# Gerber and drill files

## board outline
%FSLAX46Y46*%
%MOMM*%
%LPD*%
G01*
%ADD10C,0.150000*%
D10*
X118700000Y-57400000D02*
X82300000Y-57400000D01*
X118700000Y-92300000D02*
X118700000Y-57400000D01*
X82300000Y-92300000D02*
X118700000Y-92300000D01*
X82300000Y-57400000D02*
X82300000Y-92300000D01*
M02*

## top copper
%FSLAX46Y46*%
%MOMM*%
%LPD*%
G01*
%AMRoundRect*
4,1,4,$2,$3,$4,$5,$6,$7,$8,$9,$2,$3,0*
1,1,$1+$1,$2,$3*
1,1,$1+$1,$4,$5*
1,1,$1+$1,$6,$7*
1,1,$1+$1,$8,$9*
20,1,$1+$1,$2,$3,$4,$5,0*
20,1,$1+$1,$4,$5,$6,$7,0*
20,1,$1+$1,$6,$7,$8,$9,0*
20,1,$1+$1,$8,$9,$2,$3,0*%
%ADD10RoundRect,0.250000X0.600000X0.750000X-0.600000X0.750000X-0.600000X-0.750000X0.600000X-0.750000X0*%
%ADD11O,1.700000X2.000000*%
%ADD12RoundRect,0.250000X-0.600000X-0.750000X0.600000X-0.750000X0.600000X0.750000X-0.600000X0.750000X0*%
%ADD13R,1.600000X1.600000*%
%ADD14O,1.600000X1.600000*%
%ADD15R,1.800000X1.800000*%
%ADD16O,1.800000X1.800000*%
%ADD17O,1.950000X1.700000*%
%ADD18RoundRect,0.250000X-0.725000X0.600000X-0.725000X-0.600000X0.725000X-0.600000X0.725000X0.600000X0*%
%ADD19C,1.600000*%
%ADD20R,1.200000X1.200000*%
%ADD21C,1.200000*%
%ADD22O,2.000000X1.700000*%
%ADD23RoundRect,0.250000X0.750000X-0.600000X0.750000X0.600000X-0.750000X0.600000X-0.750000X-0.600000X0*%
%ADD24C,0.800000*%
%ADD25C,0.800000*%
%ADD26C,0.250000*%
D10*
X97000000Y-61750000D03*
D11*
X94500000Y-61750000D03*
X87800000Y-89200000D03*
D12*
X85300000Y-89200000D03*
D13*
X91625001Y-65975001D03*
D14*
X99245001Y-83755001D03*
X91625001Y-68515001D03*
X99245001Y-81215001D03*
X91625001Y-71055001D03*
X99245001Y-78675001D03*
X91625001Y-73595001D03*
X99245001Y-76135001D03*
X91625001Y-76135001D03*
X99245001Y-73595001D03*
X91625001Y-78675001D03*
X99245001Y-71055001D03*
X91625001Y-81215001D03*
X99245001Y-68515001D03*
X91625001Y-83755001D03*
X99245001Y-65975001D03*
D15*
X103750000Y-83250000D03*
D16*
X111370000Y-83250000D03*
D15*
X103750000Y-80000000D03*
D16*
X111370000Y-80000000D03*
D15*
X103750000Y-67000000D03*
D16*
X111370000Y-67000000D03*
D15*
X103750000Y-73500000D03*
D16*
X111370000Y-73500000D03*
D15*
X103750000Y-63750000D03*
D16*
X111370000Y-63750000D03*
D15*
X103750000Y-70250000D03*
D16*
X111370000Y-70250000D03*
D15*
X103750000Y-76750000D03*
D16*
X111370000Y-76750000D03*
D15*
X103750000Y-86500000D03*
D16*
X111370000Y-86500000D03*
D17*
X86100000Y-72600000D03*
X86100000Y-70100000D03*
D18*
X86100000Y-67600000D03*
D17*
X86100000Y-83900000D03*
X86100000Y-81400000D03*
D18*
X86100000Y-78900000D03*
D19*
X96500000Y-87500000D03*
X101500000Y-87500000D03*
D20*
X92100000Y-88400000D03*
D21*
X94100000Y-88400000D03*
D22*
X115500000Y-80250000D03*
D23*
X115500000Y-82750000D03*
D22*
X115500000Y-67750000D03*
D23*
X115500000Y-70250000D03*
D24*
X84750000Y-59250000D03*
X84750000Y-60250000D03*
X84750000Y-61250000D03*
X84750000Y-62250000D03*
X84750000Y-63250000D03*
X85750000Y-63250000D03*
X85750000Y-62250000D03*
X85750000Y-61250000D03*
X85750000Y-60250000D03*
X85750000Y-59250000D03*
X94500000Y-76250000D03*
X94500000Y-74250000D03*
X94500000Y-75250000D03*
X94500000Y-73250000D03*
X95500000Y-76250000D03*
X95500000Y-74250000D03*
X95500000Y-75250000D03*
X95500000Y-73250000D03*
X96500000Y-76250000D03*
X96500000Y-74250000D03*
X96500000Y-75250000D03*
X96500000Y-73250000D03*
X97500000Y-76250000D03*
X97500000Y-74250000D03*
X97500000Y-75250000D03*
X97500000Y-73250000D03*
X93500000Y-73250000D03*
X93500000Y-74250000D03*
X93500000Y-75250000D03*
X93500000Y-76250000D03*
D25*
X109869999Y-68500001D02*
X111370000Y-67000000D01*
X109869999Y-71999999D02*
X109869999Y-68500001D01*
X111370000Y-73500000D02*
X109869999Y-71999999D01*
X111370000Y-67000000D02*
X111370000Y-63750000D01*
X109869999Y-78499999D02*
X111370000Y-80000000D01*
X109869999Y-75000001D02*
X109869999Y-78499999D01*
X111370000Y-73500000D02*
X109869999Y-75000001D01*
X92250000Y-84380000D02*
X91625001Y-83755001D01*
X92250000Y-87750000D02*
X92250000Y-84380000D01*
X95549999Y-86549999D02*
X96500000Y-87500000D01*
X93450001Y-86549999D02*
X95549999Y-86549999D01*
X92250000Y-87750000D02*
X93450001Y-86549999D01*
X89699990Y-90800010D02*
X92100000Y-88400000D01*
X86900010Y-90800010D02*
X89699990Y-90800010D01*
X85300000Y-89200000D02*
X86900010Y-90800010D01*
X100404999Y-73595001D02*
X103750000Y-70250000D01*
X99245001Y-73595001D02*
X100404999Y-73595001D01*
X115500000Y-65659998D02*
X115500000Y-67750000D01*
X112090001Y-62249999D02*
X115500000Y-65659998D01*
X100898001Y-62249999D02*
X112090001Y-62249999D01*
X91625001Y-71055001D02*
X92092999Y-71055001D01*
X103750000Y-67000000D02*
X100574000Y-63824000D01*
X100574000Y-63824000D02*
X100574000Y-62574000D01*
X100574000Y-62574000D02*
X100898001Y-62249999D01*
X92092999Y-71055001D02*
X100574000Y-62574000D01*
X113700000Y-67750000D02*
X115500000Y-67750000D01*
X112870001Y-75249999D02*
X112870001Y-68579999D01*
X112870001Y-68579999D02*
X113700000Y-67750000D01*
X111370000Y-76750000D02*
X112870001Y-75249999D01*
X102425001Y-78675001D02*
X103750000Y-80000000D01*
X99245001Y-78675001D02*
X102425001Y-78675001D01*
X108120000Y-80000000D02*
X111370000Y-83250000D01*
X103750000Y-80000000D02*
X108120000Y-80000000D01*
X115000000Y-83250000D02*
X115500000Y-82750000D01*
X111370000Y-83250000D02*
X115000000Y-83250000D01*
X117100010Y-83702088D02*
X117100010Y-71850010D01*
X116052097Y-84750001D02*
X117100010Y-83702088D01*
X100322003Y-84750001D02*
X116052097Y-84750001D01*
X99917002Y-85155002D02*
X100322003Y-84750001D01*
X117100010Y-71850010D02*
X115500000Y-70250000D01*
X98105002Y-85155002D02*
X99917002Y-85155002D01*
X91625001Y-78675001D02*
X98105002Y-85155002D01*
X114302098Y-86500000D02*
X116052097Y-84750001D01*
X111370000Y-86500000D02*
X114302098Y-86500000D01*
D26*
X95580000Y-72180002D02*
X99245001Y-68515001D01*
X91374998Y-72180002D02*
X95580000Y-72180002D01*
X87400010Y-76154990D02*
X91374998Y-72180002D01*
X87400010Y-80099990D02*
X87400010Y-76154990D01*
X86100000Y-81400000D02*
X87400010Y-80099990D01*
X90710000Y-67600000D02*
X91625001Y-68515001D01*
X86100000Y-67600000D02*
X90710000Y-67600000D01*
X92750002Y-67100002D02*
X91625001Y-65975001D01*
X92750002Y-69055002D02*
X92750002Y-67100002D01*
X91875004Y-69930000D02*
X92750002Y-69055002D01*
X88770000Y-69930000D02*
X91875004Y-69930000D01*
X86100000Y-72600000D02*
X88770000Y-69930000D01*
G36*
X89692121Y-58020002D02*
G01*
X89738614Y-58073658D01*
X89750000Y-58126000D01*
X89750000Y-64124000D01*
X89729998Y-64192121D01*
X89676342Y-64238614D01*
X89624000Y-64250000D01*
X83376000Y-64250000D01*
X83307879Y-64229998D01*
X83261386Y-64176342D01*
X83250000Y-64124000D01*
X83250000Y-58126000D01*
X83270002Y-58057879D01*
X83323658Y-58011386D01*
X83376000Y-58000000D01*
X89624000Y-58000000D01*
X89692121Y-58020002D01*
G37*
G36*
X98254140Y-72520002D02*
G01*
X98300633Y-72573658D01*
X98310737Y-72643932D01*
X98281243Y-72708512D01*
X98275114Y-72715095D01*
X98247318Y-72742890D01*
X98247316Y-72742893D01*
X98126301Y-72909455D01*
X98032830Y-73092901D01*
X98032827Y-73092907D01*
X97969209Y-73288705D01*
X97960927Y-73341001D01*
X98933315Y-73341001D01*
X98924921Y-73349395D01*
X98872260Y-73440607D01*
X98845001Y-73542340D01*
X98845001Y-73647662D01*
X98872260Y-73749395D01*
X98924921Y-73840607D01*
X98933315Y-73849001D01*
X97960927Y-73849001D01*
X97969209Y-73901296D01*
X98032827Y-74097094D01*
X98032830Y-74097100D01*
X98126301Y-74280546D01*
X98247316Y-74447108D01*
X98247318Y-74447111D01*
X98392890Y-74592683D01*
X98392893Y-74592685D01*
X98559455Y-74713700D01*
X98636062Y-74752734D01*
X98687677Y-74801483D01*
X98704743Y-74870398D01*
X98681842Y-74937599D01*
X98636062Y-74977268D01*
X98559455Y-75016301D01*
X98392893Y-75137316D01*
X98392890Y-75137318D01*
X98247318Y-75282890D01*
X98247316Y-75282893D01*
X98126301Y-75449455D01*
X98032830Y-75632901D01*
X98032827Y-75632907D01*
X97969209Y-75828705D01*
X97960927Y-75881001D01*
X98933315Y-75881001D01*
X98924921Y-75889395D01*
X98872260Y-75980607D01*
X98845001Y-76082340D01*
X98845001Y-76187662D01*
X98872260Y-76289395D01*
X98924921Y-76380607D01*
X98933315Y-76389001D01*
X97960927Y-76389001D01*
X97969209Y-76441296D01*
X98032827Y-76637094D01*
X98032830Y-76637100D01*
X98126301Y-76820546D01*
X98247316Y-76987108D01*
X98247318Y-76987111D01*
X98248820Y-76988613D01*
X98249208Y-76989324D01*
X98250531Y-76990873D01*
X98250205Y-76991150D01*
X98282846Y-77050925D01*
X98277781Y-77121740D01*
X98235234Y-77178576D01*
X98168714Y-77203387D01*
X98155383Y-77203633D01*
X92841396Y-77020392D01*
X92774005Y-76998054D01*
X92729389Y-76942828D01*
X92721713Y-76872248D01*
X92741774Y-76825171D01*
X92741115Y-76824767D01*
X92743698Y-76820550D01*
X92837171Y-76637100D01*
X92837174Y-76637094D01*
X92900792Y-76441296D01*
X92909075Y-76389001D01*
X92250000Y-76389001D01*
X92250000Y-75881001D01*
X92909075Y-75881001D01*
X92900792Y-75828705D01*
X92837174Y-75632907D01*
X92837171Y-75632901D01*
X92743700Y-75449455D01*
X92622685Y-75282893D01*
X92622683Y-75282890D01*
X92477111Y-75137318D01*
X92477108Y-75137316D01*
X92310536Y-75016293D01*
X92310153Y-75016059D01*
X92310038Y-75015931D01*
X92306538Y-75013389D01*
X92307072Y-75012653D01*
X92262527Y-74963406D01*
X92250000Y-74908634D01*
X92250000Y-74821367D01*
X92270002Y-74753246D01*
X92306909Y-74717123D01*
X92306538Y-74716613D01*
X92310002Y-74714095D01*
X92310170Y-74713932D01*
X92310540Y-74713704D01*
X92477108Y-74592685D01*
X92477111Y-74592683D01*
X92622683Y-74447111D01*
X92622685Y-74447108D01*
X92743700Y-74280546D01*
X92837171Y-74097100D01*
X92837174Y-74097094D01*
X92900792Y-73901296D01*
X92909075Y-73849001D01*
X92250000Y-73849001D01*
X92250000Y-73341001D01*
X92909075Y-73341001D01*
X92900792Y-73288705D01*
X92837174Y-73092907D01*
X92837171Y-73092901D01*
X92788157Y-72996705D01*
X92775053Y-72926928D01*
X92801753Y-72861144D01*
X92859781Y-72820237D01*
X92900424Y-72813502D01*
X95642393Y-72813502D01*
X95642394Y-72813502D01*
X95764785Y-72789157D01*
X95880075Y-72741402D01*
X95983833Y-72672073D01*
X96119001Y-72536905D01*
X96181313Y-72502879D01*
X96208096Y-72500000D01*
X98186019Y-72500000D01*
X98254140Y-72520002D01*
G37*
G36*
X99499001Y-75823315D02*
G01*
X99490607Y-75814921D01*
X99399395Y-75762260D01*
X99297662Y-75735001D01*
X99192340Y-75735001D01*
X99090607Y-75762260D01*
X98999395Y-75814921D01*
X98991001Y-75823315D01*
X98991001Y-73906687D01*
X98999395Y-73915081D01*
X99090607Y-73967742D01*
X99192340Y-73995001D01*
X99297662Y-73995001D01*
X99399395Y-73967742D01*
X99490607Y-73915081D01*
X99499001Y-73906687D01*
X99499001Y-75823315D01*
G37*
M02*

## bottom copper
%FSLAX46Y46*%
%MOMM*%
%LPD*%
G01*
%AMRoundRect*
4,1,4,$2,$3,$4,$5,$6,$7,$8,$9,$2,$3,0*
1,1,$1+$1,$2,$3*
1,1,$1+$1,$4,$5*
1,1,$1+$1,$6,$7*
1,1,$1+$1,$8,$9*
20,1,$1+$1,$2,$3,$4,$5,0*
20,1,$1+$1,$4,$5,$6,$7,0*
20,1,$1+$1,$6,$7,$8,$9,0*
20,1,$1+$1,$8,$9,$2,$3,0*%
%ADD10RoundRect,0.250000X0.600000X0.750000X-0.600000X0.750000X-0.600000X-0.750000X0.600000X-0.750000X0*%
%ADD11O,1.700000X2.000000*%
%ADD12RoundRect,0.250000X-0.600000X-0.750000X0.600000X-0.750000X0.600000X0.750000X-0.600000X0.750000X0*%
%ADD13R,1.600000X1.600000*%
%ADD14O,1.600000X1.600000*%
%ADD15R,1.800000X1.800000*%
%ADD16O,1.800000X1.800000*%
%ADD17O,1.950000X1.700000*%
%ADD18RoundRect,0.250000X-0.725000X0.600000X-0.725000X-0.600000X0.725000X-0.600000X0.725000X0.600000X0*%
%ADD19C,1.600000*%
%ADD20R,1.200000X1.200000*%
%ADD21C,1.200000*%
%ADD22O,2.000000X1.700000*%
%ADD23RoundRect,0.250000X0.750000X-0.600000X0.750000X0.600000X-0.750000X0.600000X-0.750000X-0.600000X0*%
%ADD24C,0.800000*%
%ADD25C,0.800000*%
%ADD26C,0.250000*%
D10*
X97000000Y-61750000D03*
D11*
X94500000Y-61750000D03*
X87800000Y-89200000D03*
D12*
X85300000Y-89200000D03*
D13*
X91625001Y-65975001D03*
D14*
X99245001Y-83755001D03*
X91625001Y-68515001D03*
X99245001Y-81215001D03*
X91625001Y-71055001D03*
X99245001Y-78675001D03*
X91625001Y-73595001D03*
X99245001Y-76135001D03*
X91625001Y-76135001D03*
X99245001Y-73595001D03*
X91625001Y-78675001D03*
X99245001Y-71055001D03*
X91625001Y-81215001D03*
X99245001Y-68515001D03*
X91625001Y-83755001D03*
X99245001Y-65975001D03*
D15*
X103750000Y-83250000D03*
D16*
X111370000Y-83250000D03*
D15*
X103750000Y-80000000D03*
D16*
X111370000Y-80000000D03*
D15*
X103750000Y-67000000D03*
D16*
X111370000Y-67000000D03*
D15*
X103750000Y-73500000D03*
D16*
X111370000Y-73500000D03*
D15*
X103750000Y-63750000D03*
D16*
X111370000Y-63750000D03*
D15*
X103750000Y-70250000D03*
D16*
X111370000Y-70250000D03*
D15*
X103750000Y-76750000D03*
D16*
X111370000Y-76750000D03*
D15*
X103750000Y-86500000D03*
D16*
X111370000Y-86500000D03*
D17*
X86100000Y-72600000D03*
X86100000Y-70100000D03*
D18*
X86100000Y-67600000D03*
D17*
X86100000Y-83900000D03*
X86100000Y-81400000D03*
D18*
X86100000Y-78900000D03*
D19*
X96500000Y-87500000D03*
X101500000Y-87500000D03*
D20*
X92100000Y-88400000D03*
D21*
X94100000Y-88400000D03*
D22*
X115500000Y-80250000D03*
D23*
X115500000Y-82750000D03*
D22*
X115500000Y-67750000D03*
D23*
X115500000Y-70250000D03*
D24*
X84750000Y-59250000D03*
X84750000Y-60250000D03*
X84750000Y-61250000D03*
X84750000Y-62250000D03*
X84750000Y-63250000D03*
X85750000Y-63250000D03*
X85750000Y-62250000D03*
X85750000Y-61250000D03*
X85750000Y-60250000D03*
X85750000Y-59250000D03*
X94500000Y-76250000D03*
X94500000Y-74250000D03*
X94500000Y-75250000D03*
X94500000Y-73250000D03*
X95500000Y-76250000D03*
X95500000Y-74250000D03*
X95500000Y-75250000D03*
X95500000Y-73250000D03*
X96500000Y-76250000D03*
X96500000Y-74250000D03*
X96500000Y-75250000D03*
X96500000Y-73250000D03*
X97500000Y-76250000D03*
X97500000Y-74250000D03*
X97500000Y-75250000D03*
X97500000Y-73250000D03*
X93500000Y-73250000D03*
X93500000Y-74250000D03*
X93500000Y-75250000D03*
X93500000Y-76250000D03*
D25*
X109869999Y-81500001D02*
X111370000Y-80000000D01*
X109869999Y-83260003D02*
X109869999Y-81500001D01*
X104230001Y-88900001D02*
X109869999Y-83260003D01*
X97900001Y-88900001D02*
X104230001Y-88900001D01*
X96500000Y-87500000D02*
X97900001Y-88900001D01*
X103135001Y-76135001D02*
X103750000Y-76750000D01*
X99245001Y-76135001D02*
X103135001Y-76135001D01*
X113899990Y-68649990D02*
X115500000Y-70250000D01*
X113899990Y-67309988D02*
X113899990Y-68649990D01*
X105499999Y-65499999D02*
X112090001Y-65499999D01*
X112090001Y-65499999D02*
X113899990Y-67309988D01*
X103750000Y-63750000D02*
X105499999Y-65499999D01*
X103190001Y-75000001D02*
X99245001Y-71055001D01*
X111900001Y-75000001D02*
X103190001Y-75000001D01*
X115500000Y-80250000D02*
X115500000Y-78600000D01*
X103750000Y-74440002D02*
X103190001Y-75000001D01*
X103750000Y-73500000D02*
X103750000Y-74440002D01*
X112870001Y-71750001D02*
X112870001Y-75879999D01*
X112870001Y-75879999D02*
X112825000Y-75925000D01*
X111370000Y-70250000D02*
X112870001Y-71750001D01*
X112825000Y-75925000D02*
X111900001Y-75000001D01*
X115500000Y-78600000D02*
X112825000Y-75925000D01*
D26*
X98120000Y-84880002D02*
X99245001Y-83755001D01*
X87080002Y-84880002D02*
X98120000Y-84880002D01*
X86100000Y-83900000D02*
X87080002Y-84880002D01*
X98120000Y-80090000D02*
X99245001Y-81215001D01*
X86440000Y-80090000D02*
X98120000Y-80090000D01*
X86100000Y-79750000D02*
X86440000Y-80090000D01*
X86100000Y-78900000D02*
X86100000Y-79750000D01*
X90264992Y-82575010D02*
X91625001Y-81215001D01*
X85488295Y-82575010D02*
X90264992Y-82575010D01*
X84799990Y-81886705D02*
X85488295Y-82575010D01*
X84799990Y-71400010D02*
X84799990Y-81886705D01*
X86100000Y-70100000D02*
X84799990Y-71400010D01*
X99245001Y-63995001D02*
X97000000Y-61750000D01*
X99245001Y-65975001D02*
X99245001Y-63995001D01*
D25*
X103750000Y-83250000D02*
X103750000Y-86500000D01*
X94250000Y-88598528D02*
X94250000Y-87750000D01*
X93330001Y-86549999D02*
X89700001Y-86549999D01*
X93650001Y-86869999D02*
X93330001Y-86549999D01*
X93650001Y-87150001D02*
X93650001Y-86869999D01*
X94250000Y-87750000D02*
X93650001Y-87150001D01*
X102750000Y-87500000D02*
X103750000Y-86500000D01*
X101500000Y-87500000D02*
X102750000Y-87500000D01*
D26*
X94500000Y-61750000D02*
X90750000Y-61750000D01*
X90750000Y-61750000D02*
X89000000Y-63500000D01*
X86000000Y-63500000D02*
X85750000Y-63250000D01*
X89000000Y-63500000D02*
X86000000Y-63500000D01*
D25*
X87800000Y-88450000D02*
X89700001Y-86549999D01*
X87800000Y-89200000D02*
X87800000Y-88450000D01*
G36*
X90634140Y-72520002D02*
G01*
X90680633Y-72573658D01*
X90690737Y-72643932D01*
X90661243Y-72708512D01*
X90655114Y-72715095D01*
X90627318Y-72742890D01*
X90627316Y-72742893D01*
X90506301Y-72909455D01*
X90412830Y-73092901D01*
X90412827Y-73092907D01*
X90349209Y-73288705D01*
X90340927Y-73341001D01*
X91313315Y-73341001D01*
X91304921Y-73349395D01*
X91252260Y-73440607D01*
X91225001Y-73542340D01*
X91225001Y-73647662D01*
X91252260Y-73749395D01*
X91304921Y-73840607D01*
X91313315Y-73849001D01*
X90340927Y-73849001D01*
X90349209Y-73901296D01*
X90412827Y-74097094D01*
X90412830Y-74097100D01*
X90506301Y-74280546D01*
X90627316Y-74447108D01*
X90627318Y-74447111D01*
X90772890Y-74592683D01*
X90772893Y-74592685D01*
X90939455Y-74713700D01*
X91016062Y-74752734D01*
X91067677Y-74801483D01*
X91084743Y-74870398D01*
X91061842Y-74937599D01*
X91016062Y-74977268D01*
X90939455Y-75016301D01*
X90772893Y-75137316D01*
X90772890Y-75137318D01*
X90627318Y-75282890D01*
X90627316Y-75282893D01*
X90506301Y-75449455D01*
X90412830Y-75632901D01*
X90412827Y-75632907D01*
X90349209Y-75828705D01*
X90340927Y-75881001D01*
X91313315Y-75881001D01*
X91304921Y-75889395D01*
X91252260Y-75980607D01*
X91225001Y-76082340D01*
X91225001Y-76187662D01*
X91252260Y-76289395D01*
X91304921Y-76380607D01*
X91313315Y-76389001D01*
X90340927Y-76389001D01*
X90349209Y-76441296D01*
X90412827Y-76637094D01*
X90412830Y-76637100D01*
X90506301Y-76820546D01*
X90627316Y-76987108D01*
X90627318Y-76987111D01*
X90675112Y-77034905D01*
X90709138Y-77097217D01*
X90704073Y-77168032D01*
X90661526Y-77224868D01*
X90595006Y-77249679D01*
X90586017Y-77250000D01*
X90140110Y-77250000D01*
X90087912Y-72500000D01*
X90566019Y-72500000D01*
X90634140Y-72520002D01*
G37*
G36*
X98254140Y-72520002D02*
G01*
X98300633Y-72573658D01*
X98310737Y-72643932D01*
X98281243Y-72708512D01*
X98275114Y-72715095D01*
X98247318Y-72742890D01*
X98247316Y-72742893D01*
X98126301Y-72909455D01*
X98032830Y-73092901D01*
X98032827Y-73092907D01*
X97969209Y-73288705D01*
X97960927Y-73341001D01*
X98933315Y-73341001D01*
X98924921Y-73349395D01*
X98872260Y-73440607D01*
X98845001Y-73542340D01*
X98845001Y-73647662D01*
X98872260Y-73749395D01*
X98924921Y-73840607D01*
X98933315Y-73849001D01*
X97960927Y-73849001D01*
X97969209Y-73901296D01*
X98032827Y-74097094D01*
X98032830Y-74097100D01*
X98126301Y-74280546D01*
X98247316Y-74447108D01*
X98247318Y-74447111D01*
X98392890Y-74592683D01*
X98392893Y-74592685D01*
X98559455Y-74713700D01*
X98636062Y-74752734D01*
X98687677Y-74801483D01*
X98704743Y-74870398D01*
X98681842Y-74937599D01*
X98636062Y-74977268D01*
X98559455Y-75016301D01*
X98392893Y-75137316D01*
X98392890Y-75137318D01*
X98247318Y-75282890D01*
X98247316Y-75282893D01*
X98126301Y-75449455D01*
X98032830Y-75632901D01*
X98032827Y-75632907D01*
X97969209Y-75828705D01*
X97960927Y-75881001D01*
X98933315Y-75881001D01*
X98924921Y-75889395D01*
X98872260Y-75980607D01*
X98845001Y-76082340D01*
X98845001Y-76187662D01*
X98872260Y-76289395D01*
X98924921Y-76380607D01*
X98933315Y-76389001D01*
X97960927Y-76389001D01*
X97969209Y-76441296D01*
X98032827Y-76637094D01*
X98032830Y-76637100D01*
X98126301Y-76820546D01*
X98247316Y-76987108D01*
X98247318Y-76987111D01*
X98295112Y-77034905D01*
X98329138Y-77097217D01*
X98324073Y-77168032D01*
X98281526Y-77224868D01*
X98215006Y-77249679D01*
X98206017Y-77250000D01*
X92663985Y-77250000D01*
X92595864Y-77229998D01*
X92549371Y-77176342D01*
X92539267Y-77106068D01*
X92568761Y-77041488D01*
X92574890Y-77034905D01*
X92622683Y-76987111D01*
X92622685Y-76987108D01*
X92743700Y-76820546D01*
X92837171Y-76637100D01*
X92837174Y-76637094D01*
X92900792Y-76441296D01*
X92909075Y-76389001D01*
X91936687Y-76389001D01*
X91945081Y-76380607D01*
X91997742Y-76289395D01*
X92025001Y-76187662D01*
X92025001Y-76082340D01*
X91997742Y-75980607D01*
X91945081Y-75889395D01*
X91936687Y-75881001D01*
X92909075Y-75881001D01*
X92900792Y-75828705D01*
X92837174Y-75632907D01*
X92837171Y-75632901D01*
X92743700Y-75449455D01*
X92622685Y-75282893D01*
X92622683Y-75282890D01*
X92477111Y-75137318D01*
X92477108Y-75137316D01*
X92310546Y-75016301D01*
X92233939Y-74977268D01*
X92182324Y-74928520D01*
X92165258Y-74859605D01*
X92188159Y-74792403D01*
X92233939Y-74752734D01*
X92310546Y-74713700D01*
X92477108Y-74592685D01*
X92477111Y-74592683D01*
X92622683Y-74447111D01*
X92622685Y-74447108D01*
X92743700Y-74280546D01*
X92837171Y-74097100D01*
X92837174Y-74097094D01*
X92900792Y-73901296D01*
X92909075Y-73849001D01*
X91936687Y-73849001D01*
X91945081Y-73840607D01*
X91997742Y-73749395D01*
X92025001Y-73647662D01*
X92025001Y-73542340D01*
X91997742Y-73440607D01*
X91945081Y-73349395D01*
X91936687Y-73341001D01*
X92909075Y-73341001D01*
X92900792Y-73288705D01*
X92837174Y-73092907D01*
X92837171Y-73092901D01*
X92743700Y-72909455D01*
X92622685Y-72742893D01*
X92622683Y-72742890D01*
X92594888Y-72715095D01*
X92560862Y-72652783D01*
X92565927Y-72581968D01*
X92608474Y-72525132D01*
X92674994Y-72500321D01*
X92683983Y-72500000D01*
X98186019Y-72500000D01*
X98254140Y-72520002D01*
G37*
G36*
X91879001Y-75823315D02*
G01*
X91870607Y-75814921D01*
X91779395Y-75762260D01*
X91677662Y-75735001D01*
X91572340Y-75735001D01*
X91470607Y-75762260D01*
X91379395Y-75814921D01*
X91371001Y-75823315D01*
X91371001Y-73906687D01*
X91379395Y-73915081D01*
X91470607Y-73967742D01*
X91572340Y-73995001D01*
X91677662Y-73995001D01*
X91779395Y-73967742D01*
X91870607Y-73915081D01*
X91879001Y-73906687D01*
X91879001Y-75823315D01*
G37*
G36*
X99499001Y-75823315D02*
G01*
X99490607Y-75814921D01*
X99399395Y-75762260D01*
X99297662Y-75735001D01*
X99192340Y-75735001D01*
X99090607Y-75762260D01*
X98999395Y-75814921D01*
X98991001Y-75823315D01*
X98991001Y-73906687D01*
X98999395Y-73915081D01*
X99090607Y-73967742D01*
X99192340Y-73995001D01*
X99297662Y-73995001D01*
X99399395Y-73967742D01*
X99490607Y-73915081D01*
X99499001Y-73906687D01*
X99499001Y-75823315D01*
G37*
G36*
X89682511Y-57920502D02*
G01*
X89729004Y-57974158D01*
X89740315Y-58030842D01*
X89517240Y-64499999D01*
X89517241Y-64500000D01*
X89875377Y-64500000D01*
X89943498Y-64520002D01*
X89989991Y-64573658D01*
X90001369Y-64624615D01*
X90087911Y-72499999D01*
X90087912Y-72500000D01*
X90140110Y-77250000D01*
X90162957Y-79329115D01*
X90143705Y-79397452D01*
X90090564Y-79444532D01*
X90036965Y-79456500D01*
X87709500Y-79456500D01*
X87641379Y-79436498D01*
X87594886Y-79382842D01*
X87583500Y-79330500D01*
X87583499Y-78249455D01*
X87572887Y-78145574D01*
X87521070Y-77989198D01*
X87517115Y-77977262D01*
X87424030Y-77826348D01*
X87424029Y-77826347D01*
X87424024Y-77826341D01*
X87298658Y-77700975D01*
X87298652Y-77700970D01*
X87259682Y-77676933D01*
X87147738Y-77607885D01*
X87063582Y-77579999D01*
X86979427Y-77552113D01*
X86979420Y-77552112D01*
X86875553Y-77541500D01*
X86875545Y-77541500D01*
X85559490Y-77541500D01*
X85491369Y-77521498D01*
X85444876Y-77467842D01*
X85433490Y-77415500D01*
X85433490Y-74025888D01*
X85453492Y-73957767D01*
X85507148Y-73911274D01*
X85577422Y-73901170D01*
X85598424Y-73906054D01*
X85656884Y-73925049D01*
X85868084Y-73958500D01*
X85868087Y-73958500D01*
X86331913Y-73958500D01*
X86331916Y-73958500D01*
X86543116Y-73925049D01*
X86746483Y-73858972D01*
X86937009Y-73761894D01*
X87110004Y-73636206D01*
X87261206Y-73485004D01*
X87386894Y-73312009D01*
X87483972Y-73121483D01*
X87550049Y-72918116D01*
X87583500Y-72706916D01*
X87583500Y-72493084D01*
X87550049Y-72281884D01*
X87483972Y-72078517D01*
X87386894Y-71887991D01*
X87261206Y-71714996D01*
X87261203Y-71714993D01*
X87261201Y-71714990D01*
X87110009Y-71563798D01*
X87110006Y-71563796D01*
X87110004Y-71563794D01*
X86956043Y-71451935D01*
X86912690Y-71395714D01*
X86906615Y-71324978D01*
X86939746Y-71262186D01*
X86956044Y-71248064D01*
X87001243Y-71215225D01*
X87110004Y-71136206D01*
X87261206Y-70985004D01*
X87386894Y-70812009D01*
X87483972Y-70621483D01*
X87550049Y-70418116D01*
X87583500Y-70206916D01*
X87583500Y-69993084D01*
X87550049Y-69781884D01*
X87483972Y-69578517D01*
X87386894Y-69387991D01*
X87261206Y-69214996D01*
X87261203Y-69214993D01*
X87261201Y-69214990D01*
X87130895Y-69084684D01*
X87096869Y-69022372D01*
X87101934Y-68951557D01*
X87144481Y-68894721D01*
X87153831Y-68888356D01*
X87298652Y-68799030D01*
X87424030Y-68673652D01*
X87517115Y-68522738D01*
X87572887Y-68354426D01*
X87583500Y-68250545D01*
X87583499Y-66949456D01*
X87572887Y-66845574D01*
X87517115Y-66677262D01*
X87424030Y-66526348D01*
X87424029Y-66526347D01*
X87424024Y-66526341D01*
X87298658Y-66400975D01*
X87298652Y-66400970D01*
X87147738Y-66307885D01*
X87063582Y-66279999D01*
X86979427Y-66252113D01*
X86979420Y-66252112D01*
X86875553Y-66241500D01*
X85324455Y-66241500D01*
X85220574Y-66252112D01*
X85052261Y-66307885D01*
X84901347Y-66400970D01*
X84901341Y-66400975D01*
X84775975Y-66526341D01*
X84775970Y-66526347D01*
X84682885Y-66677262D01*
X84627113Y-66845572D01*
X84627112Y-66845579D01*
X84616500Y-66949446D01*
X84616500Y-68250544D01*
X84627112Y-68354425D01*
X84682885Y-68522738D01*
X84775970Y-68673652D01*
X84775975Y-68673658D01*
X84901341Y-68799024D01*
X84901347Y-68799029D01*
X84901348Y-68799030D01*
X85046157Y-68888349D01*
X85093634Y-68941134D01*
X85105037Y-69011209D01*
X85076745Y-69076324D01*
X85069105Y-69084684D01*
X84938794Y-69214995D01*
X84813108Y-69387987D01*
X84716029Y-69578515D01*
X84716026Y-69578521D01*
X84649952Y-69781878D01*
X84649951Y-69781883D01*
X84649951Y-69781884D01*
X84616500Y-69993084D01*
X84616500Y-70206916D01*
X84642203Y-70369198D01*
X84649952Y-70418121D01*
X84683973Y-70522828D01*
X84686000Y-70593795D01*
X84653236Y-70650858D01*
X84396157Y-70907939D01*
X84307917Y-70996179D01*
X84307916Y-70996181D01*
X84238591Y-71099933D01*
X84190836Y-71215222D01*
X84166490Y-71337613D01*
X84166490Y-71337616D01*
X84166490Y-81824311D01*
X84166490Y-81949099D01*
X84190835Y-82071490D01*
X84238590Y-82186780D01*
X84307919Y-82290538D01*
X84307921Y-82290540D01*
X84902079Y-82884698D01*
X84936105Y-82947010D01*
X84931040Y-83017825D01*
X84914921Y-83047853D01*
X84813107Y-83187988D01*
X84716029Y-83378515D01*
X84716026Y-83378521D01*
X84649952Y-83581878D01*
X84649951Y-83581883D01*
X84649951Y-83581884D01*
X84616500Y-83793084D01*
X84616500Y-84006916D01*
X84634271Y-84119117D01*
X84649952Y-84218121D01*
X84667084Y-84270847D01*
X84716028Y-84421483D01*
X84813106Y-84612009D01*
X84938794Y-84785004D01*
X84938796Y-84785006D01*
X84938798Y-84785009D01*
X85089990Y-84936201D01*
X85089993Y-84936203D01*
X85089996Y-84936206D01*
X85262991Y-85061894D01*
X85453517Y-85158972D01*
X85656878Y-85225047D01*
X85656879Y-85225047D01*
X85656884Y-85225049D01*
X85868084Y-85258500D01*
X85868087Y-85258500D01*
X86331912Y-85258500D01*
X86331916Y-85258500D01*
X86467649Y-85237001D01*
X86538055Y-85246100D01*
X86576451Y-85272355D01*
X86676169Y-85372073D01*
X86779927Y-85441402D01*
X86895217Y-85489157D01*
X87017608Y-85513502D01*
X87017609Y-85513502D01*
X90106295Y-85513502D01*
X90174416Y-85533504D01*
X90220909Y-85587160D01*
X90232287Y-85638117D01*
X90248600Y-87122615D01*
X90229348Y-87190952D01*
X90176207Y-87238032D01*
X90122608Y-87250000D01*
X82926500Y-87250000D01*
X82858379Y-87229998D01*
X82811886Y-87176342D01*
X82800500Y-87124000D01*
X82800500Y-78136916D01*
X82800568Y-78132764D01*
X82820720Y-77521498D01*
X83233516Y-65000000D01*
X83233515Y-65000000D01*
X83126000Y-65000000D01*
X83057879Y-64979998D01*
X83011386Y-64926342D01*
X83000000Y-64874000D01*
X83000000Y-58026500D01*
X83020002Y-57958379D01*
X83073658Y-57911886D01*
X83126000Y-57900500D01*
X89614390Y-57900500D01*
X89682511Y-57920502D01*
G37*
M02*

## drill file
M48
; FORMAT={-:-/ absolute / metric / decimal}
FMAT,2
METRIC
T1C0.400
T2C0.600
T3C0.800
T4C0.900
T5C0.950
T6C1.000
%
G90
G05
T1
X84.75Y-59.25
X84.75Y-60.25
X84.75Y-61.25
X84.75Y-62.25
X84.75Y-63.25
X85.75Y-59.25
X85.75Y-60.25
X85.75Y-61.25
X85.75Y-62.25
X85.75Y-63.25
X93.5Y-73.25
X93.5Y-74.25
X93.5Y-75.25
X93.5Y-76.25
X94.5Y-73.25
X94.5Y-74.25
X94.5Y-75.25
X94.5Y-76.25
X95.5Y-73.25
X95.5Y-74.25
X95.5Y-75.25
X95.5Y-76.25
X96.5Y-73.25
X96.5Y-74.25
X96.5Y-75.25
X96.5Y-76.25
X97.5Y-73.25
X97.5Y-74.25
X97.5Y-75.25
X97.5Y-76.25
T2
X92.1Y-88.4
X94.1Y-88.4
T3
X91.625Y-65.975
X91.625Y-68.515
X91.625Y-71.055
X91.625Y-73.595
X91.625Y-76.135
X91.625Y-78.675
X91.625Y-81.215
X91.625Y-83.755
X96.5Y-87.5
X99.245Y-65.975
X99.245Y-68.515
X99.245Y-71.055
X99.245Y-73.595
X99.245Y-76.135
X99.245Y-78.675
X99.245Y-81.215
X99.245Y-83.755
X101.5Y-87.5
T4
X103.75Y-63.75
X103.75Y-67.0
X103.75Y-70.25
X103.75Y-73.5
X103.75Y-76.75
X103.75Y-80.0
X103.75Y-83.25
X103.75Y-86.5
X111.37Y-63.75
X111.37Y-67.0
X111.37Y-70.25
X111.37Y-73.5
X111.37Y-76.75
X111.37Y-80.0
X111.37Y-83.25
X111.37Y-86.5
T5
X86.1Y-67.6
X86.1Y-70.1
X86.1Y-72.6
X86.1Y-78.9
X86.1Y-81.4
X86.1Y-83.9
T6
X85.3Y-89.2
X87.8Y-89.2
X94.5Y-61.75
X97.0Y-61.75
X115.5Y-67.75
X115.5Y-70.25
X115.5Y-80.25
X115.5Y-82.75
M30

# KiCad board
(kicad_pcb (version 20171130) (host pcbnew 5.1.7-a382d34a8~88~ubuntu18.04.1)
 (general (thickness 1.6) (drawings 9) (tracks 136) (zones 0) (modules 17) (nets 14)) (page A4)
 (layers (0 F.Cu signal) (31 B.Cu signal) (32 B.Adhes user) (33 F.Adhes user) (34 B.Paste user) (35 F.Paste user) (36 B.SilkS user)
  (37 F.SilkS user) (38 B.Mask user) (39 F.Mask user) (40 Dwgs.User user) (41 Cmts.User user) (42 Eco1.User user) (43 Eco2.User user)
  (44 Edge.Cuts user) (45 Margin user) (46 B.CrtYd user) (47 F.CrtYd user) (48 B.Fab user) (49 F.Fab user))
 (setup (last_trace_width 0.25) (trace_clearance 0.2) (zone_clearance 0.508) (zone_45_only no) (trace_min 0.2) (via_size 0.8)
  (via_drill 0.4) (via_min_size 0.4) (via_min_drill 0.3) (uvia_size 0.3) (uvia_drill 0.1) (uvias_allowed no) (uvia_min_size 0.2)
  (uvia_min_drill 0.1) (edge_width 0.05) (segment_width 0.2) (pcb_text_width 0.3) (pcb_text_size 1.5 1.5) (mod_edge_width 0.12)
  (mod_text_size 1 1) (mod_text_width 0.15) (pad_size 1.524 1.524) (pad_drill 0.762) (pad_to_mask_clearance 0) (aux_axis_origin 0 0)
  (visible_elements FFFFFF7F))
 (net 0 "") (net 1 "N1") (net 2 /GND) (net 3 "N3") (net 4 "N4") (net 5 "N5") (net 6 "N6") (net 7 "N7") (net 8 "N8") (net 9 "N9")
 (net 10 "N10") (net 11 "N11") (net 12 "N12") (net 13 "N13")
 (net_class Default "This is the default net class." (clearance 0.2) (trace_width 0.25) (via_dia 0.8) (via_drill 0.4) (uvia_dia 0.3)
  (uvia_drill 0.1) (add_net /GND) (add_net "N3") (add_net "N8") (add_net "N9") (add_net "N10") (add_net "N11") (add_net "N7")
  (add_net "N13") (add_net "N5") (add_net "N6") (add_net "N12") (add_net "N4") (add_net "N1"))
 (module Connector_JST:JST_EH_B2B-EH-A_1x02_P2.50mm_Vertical (layer F.Cu) (at 97 61.75 180)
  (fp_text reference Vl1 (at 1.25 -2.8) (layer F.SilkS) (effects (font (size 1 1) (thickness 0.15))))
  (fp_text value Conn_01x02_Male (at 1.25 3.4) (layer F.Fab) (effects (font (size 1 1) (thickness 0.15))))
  (pad 1 thru_hole roundrect (at 0 0 180) (size 1.7 2) (drill 1) (layers *.Cu *.Mask) (roundrect_rratio 0.147059) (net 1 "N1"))
  (pad 2 thru_hole oval (at 2.5 0 180) (size 1.7 2) (drill 1) (layers *.Cu *.Mask) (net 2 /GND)))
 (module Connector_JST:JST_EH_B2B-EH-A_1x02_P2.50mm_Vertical (layer F.Cu) (at 85.3 89.2)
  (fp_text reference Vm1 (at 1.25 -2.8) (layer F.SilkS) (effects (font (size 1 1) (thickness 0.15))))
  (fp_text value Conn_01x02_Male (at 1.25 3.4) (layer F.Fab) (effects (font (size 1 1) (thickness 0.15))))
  (pad 2 thru_hole oval (at 2.5 0) (size 1.7 2) (drill 1) (layers *.Cu *.Mask) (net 2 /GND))
  (pad 1 thru_hole roundrect (at 0 0) (size 1.7 2) (drill 1) (layers *.Cu *.Mask) (roundrect_rratio 0.147059) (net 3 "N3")))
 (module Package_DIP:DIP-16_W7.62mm (layer F.Cu) (at 91.625001 65.975001)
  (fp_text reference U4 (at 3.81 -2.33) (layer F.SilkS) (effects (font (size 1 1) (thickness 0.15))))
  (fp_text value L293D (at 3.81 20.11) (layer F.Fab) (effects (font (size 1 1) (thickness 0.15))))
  (pad 1 thru_hole rect (at 0 0) (size 1.6 1.6) (drill 0.8) (layers *.Cu *.Mask) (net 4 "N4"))
  (pad 9 thru_hole oval (at 7.62 17.78) (size 1.6 1.6) (drill 0.8) (layers *.Cu *.Mask) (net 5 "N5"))
  (pad 2 thru_hole oval (at 0 2.54) (size 1.6 1.6) (drill 0.8) (layers *.Cu *.Mask) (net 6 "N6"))
  (pad 10 thru_hole oval (at 7.62 15.24) (size 1.6 1.6) (drill 0.8) (layers *.Cu *.Mask) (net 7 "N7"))
  (pad 3 thru_hole oval (at 0 5.08) (size 1.6 1.6) (drill 0.8) (layers *.Cu *.Mask) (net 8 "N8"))
  (pad 11 thru_hole oval (at 7.62 12.7) (size 1.6 1.6) (drill 0.8) (layers *.Cu *.Mask) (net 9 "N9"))
  (pad 4 thru_hole oval (at 0 7.62) (size 1.6 1.6) (drill 0.8) (layers *.Cu *.Mask) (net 2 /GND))
  (pad 12 thru_hole oval (at 7.62 10.16) (size 1.6 1.6) (drill 0.8) (layers *.Cu *.Mask) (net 2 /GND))
  (pad 5 thru_hole oval (at 0 10.16) (size 1.6 1.6) (drill 0.8) (layers *.Cu *.Mask) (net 2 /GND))
  (pad 13 thru_hole oval (at 7.62 7.62) (size 1.6 1.6) (drill 0.8) (layers *.Cu *.Mask) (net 2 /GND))
  (pad 6 thru_hole oval (at 0 12.7) (size 1.6 1.6) (drill 0.8) (layers *.Cu *.Mask) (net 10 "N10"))
  (pad 14 thru_hole oval (at 7.62 5.08) (size 1.6 1.6) (drill 0.8) (layers *.Cu *.Mask) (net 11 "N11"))
  (pad 7 thru_hole oval (at 0 15.24) (size 1.6 1.6) (drill 0.8) (layers *.Cu *.Mask) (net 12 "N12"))
  (pad 15 thru_hole oval (at 7.62 2.54) (size 1.6 1.6) (drill 0.8) (layers *.Cu *.Mask) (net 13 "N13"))
  (pad 8 thru_hole oval (at 0 17.78) (size 1.6 1.6) (drill 0.8) (layers *.Cu *.Mask) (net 3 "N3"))
  (pad 16 thru_hole oval (at 7.62 0) (size 1.6 1.6) (drill 0.8) (layers *.Cu *.Mask) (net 1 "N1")))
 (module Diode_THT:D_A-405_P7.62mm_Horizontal (layer F.Cu) (at 103.75 83.25)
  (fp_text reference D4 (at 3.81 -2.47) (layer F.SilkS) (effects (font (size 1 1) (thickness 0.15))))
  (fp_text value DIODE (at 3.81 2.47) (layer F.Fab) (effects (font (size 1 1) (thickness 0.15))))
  (pad 1 thru_hole rect (at 0 0) (size 1.8 1.8) (drill 0.9) (layers *.Cu *.Mask) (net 2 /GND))
  (pad 2 thru_hole oval (at 7.62 0) (size 1.8 1.8) (drill 0.9) (layers *.Cu *.Mask) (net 9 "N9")))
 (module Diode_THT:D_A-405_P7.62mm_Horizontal (layer F.Cu) (at 103.75 80)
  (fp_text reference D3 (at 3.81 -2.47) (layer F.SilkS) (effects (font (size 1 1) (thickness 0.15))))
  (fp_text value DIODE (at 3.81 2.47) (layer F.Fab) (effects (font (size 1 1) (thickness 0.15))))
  (pad 1 thru_hole rect (at 0 0) (size 1.8 1.8) (drill 0.9) (layers *.Cu *.Mask) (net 9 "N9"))
  (pad 2 thru_hole oval (at 7.62 0) (size 1.8 1.8) (drill 0.9) (layers *.Cu *.Mask) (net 3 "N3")))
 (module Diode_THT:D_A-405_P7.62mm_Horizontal (layer F.Cu) (at 103.75 67)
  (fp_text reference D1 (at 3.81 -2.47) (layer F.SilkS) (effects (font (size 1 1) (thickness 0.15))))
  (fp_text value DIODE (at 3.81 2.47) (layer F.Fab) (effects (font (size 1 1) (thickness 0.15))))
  (pad 1 thru_hole rect (at 0 0) (size 1.8 1.8) (drill 0.9) (layers *.Cu *.Mask) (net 8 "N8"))
  (pad 2 thru_hole oval (at 7.62 0) (size 1.8 1.8) (drill 0.9) (layers *.Cu *.Mask) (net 3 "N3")))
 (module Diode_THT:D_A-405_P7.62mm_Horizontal (layer F.Cu) (at 103.75 73.5)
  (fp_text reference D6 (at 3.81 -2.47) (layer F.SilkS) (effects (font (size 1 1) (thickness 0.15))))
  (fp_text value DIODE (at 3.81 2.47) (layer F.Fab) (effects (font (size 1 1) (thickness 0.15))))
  (pad 1 thru_hole rect (at 0 0) (size 1.8 1.8) (drill 0.9) (layers *.Cu *.Mask) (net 11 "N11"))
  (pad 2 thru_hole oval (at 7.62 0) (size 1.8 1.8) (drill 0.9) (layers *.Cu *.Mask) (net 3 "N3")))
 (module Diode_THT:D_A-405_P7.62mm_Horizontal (layer F.Cu) (at 103.75 63.75)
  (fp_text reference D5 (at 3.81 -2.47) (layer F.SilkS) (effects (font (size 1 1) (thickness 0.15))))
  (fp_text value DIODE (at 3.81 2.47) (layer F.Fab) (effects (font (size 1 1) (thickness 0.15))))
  (pad 1 thru_hole rect (at 0 0) (size 1.8 1.8) (drill 0.9) (layers *.Cu *.Mask) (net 10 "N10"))
  (pad 2 thru_hole oval (at 7.62 0) (size 1.8 1.8) (drill 0.9) (layers *.Cu *.Mask) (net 3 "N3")))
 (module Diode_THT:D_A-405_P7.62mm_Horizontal (layer F.Cu) (at 103.75 70.25)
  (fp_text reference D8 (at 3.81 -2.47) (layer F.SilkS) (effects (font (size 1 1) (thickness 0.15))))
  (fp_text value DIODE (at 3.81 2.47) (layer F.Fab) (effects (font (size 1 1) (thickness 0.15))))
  (pad 1 thru_hole rect (at 0 0) (size 1.8 1.8) (drill 0.9) (layers *.Cu *.Mask) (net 2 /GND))
  (pad 2 thru_hole oval (at 7.62 0) (size 1.8 1.8) (drill 0.9) (layers *.Cu *.Mask) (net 11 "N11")))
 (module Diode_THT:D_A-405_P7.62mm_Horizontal (layer F.Cu) (at 103.75 76.75)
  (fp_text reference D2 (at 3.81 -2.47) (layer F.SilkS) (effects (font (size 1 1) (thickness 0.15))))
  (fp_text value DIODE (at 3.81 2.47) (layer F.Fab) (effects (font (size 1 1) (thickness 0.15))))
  (pad 1 thru_hole rect (at 0 0) (size 1.8 1.8) (drill 0.9) (layers *.Cu *.Mask) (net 2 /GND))
  (pad 2 thru_hole oval (at 7.62 0) (size 1.8 1.8) (drill 0.9) (layers *.Cu *.Mask) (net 8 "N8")))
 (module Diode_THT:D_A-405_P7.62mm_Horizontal (layer F.Cu) (at 103.75 86.5)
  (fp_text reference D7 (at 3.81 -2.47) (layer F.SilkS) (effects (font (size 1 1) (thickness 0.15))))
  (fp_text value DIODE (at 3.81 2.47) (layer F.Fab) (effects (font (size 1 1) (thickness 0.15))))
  (pad 1 thru_hole rect (at 0 0) (size 1.8 1.8) (drill 0.9) (layers *.Cu *.Mask) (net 2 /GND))
  (pad 2 thru_hole oval (at 7.62 0) (size 1.8 1.8) (drill 0.9) (layers *.Cu *.Mask) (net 10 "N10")))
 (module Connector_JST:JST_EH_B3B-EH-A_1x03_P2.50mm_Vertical (layer F.Cu) (at 86.1 67.6 270)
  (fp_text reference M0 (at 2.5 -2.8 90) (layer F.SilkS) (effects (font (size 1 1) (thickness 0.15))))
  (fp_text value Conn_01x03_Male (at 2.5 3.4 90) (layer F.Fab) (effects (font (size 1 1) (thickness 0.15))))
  (pad 3 thru_hole oval (at 5 0 270) (size 1.7 1.95) (drill 0.95) (layers *.Cu *.Mask) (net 4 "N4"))
  (pad 2 thru_hole oval (at 2.5 0 270) (size 1.7 1.95) (drill 0.95) (layers *.Cu *.Mask) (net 12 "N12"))
  (pad 1 thru_hole roundrect (at 0 0 270) (size 1.7 1.95) (drill 0.95) (layers *.Cu *.Mask) (roundrect_rratio 0.147059) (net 6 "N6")))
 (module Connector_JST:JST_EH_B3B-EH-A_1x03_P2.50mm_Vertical (layer F.Cu) (at 86.1 78.9 270)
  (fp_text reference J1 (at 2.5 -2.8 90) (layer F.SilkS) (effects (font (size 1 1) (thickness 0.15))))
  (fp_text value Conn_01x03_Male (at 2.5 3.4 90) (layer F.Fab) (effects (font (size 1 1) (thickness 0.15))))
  (pad 3 thru_hole oval (at 5 0 270) (size 1.7 1.95) (drill 0.95) (layers *.Cu *.Mask) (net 5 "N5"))
  (pad 2 thru_hole oval (at 2.5 0 270) (size 1.7 1.95) (drill 0.95) (layers *.Cu *.Mask) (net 13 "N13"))
  (pad 1 thru_hole roundrect (at 0 0 270) (size 1.7 1.95) (drill 0.95) (layers *.Cu *.Mask) (roundrect_rratio 0.147059) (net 7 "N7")))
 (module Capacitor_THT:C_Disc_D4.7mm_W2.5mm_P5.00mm (layer F.Cu) (at 96.5 87.5)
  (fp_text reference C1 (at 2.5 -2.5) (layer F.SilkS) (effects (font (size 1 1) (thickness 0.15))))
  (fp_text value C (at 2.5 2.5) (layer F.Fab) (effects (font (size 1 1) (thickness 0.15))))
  (pad 1 thru_hole circle (at 0 0) (size 1.6 1.6) (drill 0.8) (layers *.Cu *.Mask) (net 3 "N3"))
  (pad 2 thru_hole circle (at 5 0) (size 1.6 1.6) (drill 0.8) (layers *.Cu *.Mask) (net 2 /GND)))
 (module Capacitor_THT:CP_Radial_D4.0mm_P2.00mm (layer F.Cu) (at 92.1 88.4)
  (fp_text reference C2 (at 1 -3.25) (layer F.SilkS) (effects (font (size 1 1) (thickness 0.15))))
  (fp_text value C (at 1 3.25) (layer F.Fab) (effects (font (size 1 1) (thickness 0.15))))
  (pad 1 thru_hole rect (at 0 0) (size 1.2 1.2) (drill 0.6) (layers *.Cu *.Mask) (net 3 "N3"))
  (pad 2 thru_hole circle (at 2 0) (size 1.2 1.2) (drill 0.6) (layers *.Cu *.Mask) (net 2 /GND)))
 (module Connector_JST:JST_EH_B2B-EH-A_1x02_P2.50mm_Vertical (layer F.Cu) (at 115.5 82.75 90)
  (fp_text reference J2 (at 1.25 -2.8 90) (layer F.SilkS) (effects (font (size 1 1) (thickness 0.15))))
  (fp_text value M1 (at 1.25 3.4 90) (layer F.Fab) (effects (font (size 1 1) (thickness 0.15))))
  (pad 2 thru_hole oval (at 2.5 0 90) (size 1.7 2) (drill 1) (layers *.Cu *.Mask) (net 11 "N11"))
  (pad 1 thru_hole roundrect (at 0 0 90) (size 1.7 2) (drill 1) (layers *.Cu *.Mask) (roundrect_rratio 0.147059) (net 9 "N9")))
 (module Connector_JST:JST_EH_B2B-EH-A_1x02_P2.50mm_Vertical (layer F.Cu) (at 115.5 70.25 90)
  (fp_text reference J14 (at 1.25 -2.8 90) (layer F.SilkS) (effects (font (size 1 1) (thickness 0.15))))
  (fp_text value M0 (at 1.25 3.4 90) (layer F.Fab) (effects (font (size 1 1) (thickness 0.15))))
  (pad 2 thru_hole oval (at 2.5 0 90) (size 1.7 2) (drill 1) (layers *.Cu *.Mask) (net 8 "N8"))
  (pad 1 thru_hole roundrect (at 0 0 90) (size 1.7 2) (drill 1) (layers *.Cu *.Mask) (roundrect_rratio 0.147059) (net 10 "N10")))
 (gr_line (start 118.7 57.4) (end 82.3 57.4) (layer Edge.Cuts) (width 0.15))
 (gr_line (start 118.7 92.3) (end 118.7 57.4) (layer Edge.Cuts) (width 0.15))
 (gr_line (start 82.3 92.3) (end 118.7 92.3) (layer Edge.Cuts) (width 0.15))
 (gr_line (start 82.3 57.4) (end 82.3 92.3) (layer Edge.Cuts) (width 0.15))
 (via (at 84.75 59.25) (size 0.8) (drill 0.4) (layers F.Cu B.Cu) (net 2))
 (via (at 84.75 60.25) (size 0.8) (drill 0.4) (layers F.Cu B.Cu) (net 2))
 (via (at 84.75 61.25) (size 0.8) (drill 0.4) (layers F.Cu B.Cu) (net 2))
 (via (at 84.75 62.25) (size 0.8) (drill 0.4) (layers F.Cu B.Cu) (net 2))
 (via (at 84.75 63.25) (size 0.8) (drill 0.4) (layers F.Cu B.Cu) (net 2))
 (via (at 85.75 63.25) (size 0.8) (drill 0.4) (layers F.Cu B.Cu) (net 2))
 (via (at 85.75 62.25) (size 0.8) (drill 0.4) (layers F.Cu B.Cu) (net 2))
 (via (at 85.75 61.25) (size 0.8) (drill 0.4) (layers F.Cu B.Cu) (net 2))
 (via (at 85.75 60.25) (size 0.8) (drill 0.4) (layers F.Cu B.Cu) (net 2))
 (via (at 85.75 59.25) (size 0.8) (drill 0.4) (layers F.Cu B.Cu) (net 2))
 (via (at 94.5 76.25) (size 0.8) (drill 0.4) (layers F.Cu B.Cu) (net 2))
 (via (at 94.5 74.25) (size 0.8) (drill 0.4) (layers F.Cu B.Cu) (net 2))
 (via (at 94.5 75.25) (size 0.8) (drill 0.4) (layers F.Cu B.Cu) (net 2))
 (via (at 94.5 73.25) (size 0.8) (drill 0.4) (layers F.Cu B.Cu) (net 2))
 (via (at 95.5 76.25) (size 0.8) (drill 0.4) (layers F.Cu B.Cu) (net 2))
 (via (at 95.5 74.25) (size 0.8) (drill 0.4) (layers F.Cu B.Cu) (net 2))
 (via (at 95.5 75.25) (size 0.8) (drill 0.4) (layers F.Cu B.Cu) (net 2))
 (via (at 95.5 73.25) (size 0.8) (drill 0.4) (layers F.Cu B.Cu) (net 2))
 (via (at 96.5 76.25) (size 0.8) (drill 0.4) (layers F.Cu B.Cu) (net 2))
 (via (at 96.5 74.25) (size 0.8) (drill 0.4) (layers F.Cu B.Cu) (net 2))
 (via (at 96.5 75.25) (size 0.8) (drill 0.4) (layers F.Cu B.Cu) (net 2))
 (via (at 96.5 73.25) (size 0.8) (drill 0.4) (layers F.Cu B.Cu) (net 2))
 (via (at 97.5 76.25) (size 0.8) (drill 0.4) (layers F.Cu B.Cu) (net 2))
 (via (at 97.5 74.25) (size 0.8) (drill 0.4) (layers F.Cu B.Cu) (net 2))
 (via (at 97.5 75.25) (size 0.8) (drill 0.4) (layers F.Cu B.Cu) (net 2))
 (via (at 97.5 73.25) (size 0.8) (drill 0.4) (layers F.Cu B.Cu) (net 2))
 (segment (start 109.869999 68.500001) (end 111.37 67) (width 0.8) (layer F.Cu) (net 3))
 (segment (start 109.869999 71.999999) (end 109.869999 68.500001) (width 0.8) (layer F.Cu) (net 3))
 (segment (start 111.37 73.5) (end 109.869999 71.999999) (width 0.8) (layer F.Cu) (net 3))
 (segment (start 111.37 67) (end 111.37 63.75) (width 0.8) (layer F.Cu) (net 3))
 (segment (start 109.869999 78.499999) (end 111.37 80) (width 0.8) (layer F.Cu) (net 3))
 (segment (start 109.869999 75.000001) (end 109.869999 78.499999) (width 0.8) (layer F.Cu) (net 3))
 (segment (start 111.37 73.5) (end 109.869999 75.000001) (width 0.8) (layer F.Cu) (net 3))
 (segment (start 92.25 84.38) (end 91.625001 83.755001) (width 0.8) (layer F.Cu) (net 3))
 (segment (start 92.25 87.75) (end 92.25 84.38) (width 0.8) (layer F.Cu) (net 3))
 (segment (start 95.549999 86.549999) (end 96.5 87.5) (width 0.8) (layer F.Cu) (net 3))
 (segment (start 93.450001 86.549999) (end 95.549999 86.549999) (width 0.8) (layer F.Cu) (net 3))
 (segment (start 92.25 87.75) (end 93.450001 86.549999) (width 0.8) (layer F.Cu) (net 3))
 (segment (start 109.869999 81.500001) (end 111.37 80) (width 0.8) (layer B.Cu) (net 3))
 (segment (start 109.869999 83.260003) (end 109.869999 81.500001) (width 0.8) (layer B.Cu) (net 3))
 (segment (start 104.230001 88.900001) (end 109.869999 83.260003) (width 0.8) (layer B.Cu) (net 3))
 (segment (start 97.900001 88.900001) (end 104.230001 88.900001) (width 0.8) (layer B.Cu) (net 3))
 (segment (start 96.5 87.5) (end 97.900001 88.900001) (width 0.8) (layer B.Cu) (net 3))
 (segment (start 89.69999 90.80001) (end 92.1 88.4) (width 0.8) (layer F.Cu) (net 3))
 (segment (start 86.90001 90.80001) (end 89.69999 90.80001) (width 0.8) (layer F.Cu) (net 3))
 (segment (start 85.3 89.2) (end 86.90001 90.80001) (width 0.8) (layer F.Cu) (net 3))
 (segment (start 100.404999 73.595001) (end 103.75 70.25) (width 0.8) (layer F.Cu) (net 2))
 (segment (start 99.245001 73.595001) (end 100.404999 73.595001) (width 0.8) (layer F.Cu) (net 2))
 (segment (start 103.135001 76.135001) (end 103.75 76.75) (width 0.8) (layer B.Cu) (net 2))
 (segment (start 99.245001 76.135001) (end 103.135001 76.135001) (width 0.8) (layer B.Cu) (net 2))
 (segment (start 115.5 65.659998) (end 115.5 67.75) (width 0.8) (layer F.Cu) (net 8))
 (segment (start 112.090001 62.249999) (end 115.5 65.659998) (width 0.8) (layer F.Cu) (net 8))
 (segment (start 100.898001 62.249999) (end 112.090001 62.249999) (width 0.8) (layer F.Cu) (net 8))
 (segment (start 91.625001 71.055001) (end 92.092999 71.055001) (width 0.8) (layer F.Cu) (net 8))
 (segment (start 103.75 67) (end 100.574 63.824) (width 0.8) (layer F.Cu) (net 8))
 (segment (start 100.574 63.824) (end 100.574 62.574) (width 0.8) (layer F.Cu) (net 8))
 (segment (start 100.574 62.574) (end 100.898001 62.249999) (width 0.8) (layer F.Cu) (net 8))
 (segment (start 92.092999 71.055001) (end 100.574 62.574) (width 0.8) (layer F.Cu) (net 8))
 (segment (start 113.7 67.75) (end 115.5 67.75) (width 0.8) (layer F.Cu) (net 8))
 (segment (start 112.870001 75.249999) (end 112.870001 68.579999) (width 0.8) (layer F.Cu) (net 8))
 (segment (start 112.870001 68.579999) (end 113.7 67.75) (width 0.8) (layer F.Cu) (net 8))
 (segment (start 111.37 76.75) (end 112.870001 75.249999) (width 0.8) (layer F.Cu) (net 8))
 (segment (start 102.425001 78.675001) (end 103.75 80) (width 0.8) (layer F.Cu) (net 9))
 (segment (start 99.245001 78.675001) (end 102.425001 78.675001) (width 0.8) (layer F.Cu) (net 9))
 (segment (start 108.12 80) (end 111.37 83.25) (width 0.8) (layer F.Cu) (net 9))
 (segment (start 103.75 80) (end 108.12 80) (width 0.8) (layer F.Cu) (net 9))
 (segment (start 115 83.25) (end 115.5 82.75) (width 0.8) (layer F.Cu) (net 9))
 (segment (start 111.37 83.25) (end 115 83.25) (width 0.8) (layer F.Cu) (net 9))
 (segment (start 117.10001 83.702088) (end 117.10001 71.85001) (width 0.8) (layer F.Cu) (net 10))
 (segment (start 116.052097 84.750001) (end 117.10001 83.702088) (width 0.8) (layer F.Cu) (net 10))
 (segment (start 100.322003 84.750001) (end 116.052097 84.750001) (width 0.8) (layer F.Cu) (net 10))
 (segment (start 99.917002 85.155002) (end 100.322003 84.750001) (width 0.8) (layer F.Cu) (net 10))
 (segment (start 117.10001 71.85001) (end 115.5 70.25) (width 0.8) (layer F.Cu) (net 10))
 (segment (start 98.105002 85.155002) (end 99.917002 85.155002) (width 0.8) (layer F.Cu) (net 10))
 (segment (start 91.625001 78.675001) (end 98.105002 85.155002) (width 0.8) (layer F.Cu) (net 10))
 (segment (start 113.89999 68.64999) (end 115.5 70.25) (width 0.8) (layer B.Cu) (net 10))
 (segment (start 113.89999 67.309988) (end 113.89999 68.64999) (width 0.8) (layer B.Cu) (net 10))
 (segment (start 105.499999 65.499999) (end 112.090001 65.499999) (width 0.8) (layer B.Cu) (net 10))
 (segment (start 112.090001 65.499999) (end 113.89999 67.309988) (width 0.8) (layer B.Cu) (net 10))
 (segment (start 103.75 63.75) (end 105.499999 65.499999) (width 0.8) (layer B.Cu) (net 10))
 (segment (start 114.302098 86.5) (end 116.052097 84.750001) (width 0.8) (layer F.Cu) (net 10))
 (segment (start 111.37 86.5) (end 114.302098 86.5) (width 0.8) (layer F.Cu) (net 10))
 (segment (start 103.190001 75.000001) (end 99.245001 71.055001) (width 0.8) (layer B.Cu) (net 11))
 (segment (start 111.900001 75.000001) (end 103.190001 75.000001) (width 0.8) (layer B.Cu) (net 11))
 (segment (start 115.5 80.25) (end 115.5 78.6) (width 0.8) (layer B.Cu) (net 11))
 (segment (start 103.75 74.440002) (end 103.190001 75.000001) (width 0.8) (layer B.Cu) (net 11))
 (segment (start 103.75 73.5) (end 103.75 74.440002) (width 0.8) (layer B.Cu) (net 11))
 (segment (start 112.870001 71.750001) (end 112.870001 75.879999) (width 0.8) (layer B.Cu) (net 11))
 (segment (start 112.870001 75.879999) (end 112.825 75.925) (width 0.8) (layer B.Cu) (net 11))
 (segment (start 111.37 70.25) (end 112.870001 71.750001) (width 0.8) (layer B.Cu) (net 11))
 (segment (start 112.825 75.925) (end 111.900001 75.000001) (width 0.8) (layer B.Cu) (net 11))
 (segment (start 115.5 78.6) (end 112.825 75.925) (width 0.8) (layer B.Cu) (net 11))
 (segment (start 98.12 84.880002) (end 99.245001 83.755001) (width 0.25) (layer B.Cu) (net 5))
 (segment (start 87.080002 84.880002) (end 98.12 84.880002) (width 0.25) (layer B.Cu) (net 5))
 (segment (start 86.1 83.9) (end 87.080002 84.880002) (width 0.25) (layer B.Cu) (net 5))
 (segment (start 95.58 72.180002) (end 99.245001 68.515001) (width 0.25) (layer F.Cu) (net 13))
 (segment (start 91.374998 72.180002) (end 95.58 72.180002) (width 0.25) (layer F.Cu) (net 13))
 (segment (start 87.40001 76.15499) (end 91.374998 72.180002) (width 0.25) (layer F.Cu) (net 13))
 (segment (start 87.40001 80.09999) (end 87.40001 76.15499) (width 0.25) (layer F.Cu) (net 13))
 (segment (start 86.1 81.4) (end 87.40001 80.09999) (width 0.25) (layer F.Cu) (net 13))
 (segment (start 98.12 80.09) (end 99.245001 81.215001) (width 0.25) (layer B.Cu) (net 7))
 (segment (start 86.44 80.09) (end 98.12 80.09) (width 0.25) (layer B.Cu) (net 7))
 (segment (start 86.1 79.75) (end 86.44 80.09) (width 0.25) (layer B.Cu) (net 7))
 (segment (start 86.1 78.9) (end 86.1 79.75) (width 0.25) (layer B.Cu) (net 7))
 (segment (start 90.71 67.6) (end 91.625001 68.515001) (width 0.25) (layer F.Cu) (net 6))
 (segment (start 86.1 67.6) (end 90.71 67.6) (width 0.25) (layer F.Cu) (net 6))
 (segment (start 90.264992 82.57501) (end 91.625001 81.215001) (width 0.25) (layer B.Cu) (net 12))
 (segment (start 85.488295 82.57501) (end 90.264992 82.57501) (width 0.25) (layer B.Cu) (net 12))
 (segment (start 84.79999 81.886705) (end 85.488295 82.57501) (width 0.25) (layer B.Cu) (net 12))
 (segment (start 84.79999 71.40001) (end 84.79999 81.886705) (width 0.25) (layer B.Cu) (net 12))
 (segment (start 86.1 70.1) (end 84.79999 71.40001) (width 0.25) (layer B.Cu) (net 12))
 (segment (start 92.750002 67.100002) (end 91.625001 65.975001) (width 0.25) (layer F.Cu) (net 4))
 (segment (start 92.750002 69.055002) (end 92.750002 67.100002) (width 0.25) (layer F.Cu) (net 4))
 (segment (start 91.875004 69.93) (end 92.750002 69.055002) (width 0.25) (layer F.Cu) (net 4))
 (segment (start 88.77 69.93) (end 91.875004 69.93) (width 0.25) (layer F.Cu) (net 4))
 (segment (start 86.1 72.6) (end 88.77 69.93) (width 0.25) (layer F.Cu) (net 4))
 (segment (start 99.245001 63.995001) (end 97 61.75) (width 0.25) (layer B.Cu) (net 1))
 (segment (start 99.245001 65.975001) (end 99.245001 63.995001) (width 0.25) (layer B.Cu) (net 1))
 (via (at 93.5 73.25) (size 0.8) (drill 0.4) (layers F.Cu B.Cu) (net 2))
 (via (at 93.5 74.25) (size 0.8) (drill 0.4) (layers F.Cu B.Cu) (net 2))
 (via (at 93.5 75.25) (size 0.8) (drill 0.4) (layers F.Cu B.Cu) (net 2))
 (via (at 93.5 76.25) (size 0.8) (drill 0.4) (layers F.Cu B.Cu) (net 2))
 (segment (start 103.75 83.25) (end 103.75 86.5) (width 0.8) (layer B.Cu) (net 2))
 (segment (start 94.25 88.598528) (end 94.25 87.75) (width 0.8) (layer B.Cu) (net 2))
 (segment (start 93.330001 86.549999) (end 89.700001 86.549999) (width 0.8) (layer B.Cu) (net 2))
 (segment (start 93.650001 86.869999) (end 93.330001 86.549999) (width 0.8) (layer B.Cu) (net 2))
 (segment (start 93.650001 87.150001) (end 93.650001 86.869999) (width 0.8) (layer B.Cu) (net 2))
 (segment (start 94.25 87.75) (end 93.650001 87.150001) (width 0.8) (layer B.Cu) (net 2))
 (segment (start 102.75 87.5) (end 103.75 86.5) (width 0.8) (layer B.Cu) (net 2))
 (segment (start 101.5 87.5) (end 102.75 87.5) (width 0.8) (layer B.Cu) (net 2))
 (segment (start 94.5 61.75) (end 90.75 61.75) (width 0.25) (layer B.Cu) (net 2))
 (segment (start 90.75 61.75) (end 89 63.5) (width 0.25) (layer B.Cu) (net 2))
 (segment (start 86 63.5) (end 85.75 63.25) (width 0.25) (layer B.Cu) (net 2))
 (segment (start 89 63.5) (end 86 63.5) (width 0.25) (layer B.Cu) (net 2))
 (segment (start 87.8 88.45) (end 89.700001 86.549999) (width 0.8) (layer B.Cu) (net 2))
 (segment (start 87.8 89.2) (end 87.8 88.45) (width 0.8) (layer B.Cu) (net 2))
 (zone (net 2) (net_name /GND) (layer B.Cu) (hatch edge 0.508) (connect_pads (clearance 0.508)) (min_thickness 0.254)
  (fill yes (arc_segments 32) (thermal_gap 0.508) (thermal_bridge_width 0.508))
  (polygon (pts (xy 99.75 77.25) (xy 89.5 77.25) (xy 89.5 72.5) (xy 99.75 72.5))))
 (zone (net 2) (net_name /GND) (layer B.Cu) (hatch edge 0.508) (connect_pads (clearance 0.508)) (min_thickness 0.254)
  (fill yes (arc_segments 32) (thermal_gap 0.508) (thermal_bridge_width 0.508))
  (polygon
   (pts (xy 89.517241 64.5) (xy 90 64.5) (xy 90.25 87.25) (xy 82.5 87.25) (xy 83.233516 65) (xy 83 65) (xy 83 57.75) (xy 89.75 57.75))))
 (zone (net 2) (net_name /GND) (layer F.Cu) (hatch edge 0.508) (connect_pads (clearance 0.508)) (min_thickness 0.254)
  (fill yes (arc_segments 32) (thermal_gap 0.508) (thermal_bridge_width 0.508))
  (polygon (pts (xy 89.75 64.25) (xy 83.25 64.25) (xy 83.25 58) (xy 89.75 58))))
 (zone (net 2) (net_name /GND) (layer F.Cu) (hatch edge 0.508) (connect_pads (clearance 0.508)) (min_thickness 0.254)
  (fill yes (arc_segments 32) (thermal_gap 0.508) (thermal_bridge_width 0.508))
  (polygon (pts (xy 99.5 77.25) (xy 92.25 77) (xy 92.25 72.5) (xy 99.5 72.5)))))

